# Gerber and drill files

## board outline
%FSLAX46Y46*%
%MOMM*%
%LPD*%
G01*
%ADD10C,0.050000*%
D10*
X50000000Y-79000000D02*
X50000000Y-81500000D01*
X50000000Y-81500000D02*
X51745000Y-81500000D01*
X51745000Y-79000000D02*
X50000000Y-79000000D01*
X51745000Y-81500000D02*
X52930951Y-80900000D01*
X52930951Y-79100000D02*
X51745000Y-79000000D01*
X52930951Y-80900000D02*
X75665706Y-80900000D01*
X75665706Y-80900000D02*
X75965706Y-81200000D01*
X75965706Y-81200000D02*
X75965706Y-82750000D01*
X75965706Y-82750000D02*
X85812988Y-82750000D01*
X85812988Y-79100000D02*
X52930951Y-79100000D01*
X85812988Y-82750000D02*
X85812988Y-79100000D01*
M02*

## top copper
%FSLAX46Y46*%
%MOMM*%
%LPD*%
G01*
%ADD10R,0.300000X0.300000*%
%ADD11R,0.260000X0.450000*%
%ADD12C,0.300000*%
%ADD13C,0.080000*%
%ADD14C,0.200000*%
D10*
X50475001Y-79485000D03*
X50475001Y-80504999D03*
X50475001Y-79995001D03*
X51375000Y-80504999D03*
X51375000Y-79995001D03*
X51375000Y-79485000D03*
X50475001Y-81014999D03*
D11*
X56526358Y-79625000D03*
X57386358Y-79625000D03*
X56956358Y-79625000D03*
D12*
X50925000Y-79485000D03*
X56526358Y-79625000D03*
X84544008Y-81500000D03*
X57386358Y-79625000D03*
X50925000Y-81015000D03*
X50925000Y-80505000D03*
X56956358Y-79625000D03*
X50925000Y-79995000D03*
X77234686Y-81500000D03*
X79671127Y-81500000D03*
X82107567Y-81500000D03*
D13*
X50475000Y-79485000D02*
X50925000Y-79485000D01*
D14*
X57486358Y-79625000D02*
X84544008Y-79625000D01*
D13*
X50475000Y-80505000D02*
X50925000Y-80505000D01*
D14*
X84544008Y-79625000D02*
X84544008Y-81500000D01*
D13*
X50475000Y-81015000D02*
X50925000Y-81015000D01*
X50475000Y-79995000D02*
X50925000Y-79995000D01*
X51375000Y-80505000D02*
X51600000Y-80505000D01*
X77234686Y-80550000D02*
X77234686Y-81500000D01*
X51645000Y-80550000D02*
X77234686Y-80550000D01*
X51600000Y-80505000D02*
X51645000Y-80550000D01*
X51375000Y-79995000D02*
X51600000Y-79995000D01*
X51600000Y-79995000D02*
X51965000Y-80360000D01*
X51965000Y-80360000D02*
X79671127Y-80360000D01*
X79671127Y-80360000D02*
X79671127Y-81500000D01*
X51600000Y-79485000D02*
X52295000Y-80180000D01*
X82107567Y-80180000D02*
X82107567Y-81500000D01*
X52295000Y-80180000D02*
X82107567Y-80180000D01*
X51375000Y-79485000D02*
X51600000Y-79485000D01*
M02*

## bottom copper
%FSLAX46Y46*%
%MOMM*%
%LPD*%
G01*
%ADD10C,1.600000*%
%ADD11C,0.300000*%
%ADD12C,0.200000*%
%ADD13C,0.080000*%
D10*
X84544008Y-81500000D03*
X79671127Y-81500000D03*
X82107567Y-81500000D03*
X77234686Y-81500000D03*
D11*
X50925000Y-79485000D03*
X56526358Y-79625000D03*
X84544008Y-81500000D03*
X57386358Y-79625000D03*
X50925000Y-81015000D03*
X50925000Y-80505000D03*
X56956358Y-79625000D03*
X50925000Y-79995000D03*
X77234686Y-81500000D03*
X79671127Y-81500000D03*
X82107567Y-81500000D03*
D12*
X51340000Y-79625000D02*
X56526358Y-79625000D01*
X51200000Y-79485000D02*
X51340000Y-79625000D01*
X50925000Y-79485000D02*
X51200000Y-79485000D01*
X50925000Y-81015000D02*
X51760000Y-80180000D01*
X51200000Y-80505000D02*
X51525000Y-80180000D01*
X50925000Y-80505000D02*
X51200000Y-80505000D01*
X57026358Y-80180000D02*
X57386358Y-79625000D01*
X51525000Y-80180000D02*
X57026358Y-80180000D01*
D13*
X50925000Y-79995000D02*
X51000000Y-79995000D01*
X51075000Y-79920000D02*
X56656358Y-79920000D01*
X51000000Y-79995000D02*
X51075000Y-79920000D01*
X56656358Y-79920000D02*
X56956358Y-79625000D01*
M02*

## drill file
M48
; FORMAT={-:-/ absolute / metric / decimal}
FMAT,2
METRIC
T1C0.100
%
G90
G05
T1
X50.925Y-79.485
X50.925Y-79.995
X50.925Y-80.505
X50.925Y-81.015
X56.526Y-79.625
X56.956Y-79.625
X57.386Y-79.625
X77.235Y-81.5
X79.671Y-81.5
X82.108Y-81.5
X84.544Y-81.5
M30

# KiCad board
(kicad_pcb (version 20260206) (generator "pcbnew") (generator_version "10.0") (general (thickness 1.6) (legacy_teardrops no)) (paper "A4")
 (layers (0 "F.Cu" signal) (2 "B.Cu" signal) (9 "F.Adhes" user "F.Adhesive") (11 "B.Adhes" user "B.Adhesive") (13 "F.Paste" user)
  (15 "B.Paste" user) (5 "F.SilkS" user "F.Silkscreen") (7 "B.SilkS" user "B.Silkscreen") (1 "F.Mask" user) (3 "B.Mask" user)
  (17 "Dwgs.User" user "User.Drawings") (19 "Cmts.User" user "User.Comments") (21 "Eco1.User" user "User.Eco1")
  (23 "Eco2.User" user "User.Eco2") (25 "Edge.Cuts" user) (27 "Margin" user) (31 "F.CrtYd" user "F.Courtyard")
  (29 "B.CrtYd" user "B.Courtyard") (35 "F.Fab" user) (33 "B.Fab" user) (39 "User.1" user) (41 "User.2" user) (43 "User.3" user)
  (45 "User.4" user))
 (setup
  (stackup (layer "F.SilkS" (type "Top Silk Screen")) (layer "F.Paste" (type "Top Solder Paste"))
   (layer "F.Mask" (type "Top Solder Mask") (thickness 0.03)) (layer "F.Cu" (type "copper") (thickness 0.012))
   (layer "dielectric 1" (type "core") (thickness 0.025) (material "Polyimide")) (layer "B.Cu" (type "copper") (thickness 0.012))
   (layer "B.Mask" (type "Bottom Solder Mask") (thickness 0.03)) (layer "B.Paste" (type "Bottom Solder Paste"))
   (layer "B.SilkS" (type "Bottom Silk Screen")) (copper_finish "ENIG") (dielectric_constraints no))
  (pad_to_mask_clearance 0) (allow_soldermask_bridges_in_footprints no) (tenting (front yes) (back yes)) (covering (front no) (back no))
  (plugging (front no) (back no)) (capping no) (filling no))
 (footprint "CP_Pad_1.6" (layer "F.Cu") (at 84.544008 81.5)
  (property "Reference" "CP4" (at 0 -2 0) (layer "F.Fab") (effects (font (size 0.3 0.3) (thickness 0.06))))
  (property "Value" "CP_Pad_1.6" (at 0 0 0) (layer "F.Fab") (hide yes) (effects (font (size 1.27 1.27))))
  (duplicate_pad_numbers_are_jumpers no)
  (pad "1" smd circle (at 0 0) (size 1.6 1.6) (layers "B.Cu" "B.Mask") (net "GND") (solder_mask_margin 0.1)))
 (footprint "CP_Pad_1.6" (layer "F.Cu") (at 77.234686 81.5)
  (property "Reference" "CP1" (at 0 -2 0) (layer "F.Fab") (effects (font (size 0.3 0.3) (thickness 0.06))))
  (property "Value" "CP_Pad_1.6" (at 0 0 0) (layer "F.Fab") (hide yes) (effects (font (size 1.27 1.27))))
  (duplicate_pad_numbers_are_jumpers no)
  (pad "1" smd circle (at 0 0) (size 1.6 1.6) (layers "B.Cu" "B.Mask") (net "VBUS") (solder_mask_margin 0.1)))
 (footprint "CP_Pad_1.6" (layer "F.Cu") (at 82.107567 81.5)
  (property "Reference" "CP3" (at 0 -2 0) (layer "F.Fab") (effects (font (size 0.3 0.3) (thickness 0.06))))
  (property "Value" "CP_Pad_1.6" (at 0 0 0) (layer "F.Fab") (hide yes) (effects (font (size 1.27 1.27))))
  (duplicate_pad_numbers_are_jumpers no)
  (pad "1" smd circle (at 0 0) (size 1.6 1.6) (layers "B.Cu" "B.Mask") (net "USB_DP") (solder_mask_margin 0.1)))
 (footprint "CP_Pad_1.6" (layer "F.Cu") (at 79.671127 81.5)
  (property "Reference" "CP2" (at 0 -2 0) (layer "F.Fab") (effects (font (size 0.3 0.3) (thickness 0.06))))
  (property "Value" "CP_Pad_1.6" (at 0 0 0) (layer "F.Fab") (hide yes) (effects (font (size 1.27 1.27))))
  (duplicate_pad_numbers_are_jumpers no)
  (pad "1" smd circle (at 0 0) (size 1.6 1.6) (layers "B.Cu" "B.Mask") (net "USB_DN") (solder_mask_margin 0.1)))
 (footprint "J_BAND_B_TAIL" (layer "F.Cu") (at 50.9 80.25)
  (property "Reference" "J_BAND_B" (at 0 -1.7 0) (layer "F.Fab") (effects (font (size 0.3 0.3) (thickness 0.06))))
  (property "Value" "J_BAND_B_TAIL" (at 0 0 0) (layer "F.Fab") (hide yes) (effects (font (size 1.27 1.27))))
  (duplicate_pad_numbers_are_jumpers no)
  (pad "1" smd rect (at -0.424999 -0.765) (size 0.3 0.3) (layers "F.Cu" "F.Mask") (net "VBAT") (solder_mask_margin 0.05)
   (thermal_bridge_angle 45))
  (pad "2" smd rect (at -0.424999 0.254999) (size 0.3 0.3) (layers "F.Cu" "F.Mask") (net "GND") (solder_mask_margin 0.05)
   (thermal_bridge_angle 45))
  (pad "3" smd rect (at -0.424999 -0.254999) (size 0.3 0.3) (layers "F.Cu" "F.Mask") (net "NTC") (solder_mask_margin 0.05)
   (thermal_bridge_angle 45))
  (pad "4" smd rect (at 0.475 0.254999) (size 0.3 0.3) (layers "F.Cu" "F.Mask") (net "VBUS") (solder_mask_margin 0.05)
   (thermal_bridge_angle 45))
  (pad "5" smd rect (at 0.475 -0.254999) (size 0.3 0.3) (layers "F.Cu" "F.Mask") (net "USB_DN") (solder_mask_margin 0.05)
   (thermal_bridge_angle 45))
  (pad "6" smd rect (at 0.475 -0.765) (size 0.3 0.3) (layers "F.Cu" "F.Mask") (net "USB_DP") (solder_mask_margin 0.05)
   (thermal_bridge_angle 45))
  (pad "7" smd rect (at -0.424999 0.764999) (size 0.3 0.3) (layers "F.Cu" "F.Mask") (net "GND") (solder_mask_margin 0.05)
   (thermal_bridge_angle 45)))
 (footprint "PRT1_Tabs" (layer "F.Cu") (at 56.956358 79.625)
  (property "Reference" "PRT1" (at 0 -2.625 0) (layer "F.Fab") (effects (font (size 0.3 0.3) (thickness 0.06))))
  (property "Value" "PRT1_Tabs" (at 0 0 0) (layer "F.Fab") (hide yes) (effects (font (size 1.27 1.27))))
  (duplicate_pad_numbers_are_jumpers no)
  (pad "1" smd rect (at -0.43 0) (size 0.26 0.45) (layers "F.Cu" "F.Mask") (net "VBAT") (solder_mask_margin 0.05) (thermal_bridge_angle 45))
  (pad "2" smd rect (at 0.43 0) (size 0.26 0.45) (layers "F.Cu" "F.Mask") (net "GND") (solder_mask_margin 0.05) (thermal_bridge_angle 45))
  (pad "3" smd rect (at 0 0) (size 0.26 0.45) (layers "F.Cu" "F.Mask") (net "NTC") (solder_mask_margin 0.05) (thermal_bridge_angle 45)))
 (gr_line (start 50 79) (end 50 81.5) (stroke (width 0.05) (type default)) (layer "Edge.Cuts"))
 (gr_line (start 50 81.5) (end 51.745 81.5) (stroke (width 0.05) (type default)) (layer "Edge.Cuts"))
 (gr_line (start 51.745 79) (end 50 79) (stroke (width 0.05) (type default)) (layer "Edge.Cuts"))
 (gr_line (start 51.745 81.5) (end 52.930951 80.9) (stroke (width 0.05) (type default)) (layer "Edge.Cuts"))
 (gr_line (start 52.930951 79.1) (end 51.745 79) (stroke (width 0.05) (type default)) (layer "Edge.Cuts"))
 (gr_line (start 52.930951 80.9) (end 75.665706 80.9) (stroke (width 0.05) (type default)) (layer "Edge.Cuts"))
 (gr_line (start 75.665706 80.9) (end 75.965706 81.2) (stroke (width 0.05) (type default)) (layer "Edge.Cuts"))
 (gr_line (start 75.965706 81.2) (end 75.965706 82.75) (stroke (width 0.05) (type default)) (layer "Edge.Cuts"))
 (gr_line (start 75.965706 82.75) (end 85.812988 82.75) (stroke (width 0.05) (type default)) (layer "Edge.Cuts"))
 (gr_line (start 85.812988 79.1) (end 52.930951 79.1) (stroke (width 0.05) (type default)) (layer "Edge.Cuts"))
 (gr_line (start 85.812988 82.75) (end 85.812988 79.1) (stroke (width 0.05) (type default)) (layer "Edge.Cuts"))
 (segment (start 50.475 79.485) (end 50.925 79.485) (width 0.08) (layer "F.Cu") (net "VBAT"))
 (via (at 56.526358 79.625) (size 0.3) (drill 0.1) (layers "F.Cu" "B.Cu") (tenting (front yes) (back yes)) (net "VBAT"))
 (via (at 50.925 79.485) (size 0.3) (drill 0.1) (layers "F.Cu" "B.Cu") (tenting (front yes) (back yes)) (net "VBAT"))
 (segment (start 50.925 79.485) (end 51.2 79.485) (width 0.2) (layer "B.Cu") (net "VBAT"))
 (segment (start 51.34 79.625) (end 56.526358 79.625) (width 0.2) (layer "B.Cu") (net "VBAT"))
 (segment (start 51.2 79.485) (end 51.34 79.625) (width 0.2) (layer "B.Cu") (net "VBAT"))
 (segment (start 50.475 81.015) (end 50.925 81.015) (width 0.08) (layer "F.Cu") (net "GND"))
 (segment (start 84.544008 79.625) (end 84.544008 81.5) (width 0.2) (layer "F.Cu") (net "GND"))
 (segment (start 50.475 80.505) (end 50.925 80.505) (width 0.08) (layer "F.Cu") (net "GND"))
 (segment (start 57.486358 79.625) (end 84.544008 79.625) (width 0.2) (layer "F.Cu") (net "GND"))
 (via (at 50.925 81.015) (size 0.3) (drill 0.1) (layers "F.Cu" "B.Cu") (tenting (front yes) (back yes)) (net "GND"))
 (via (at 57.386358 79.625) (size 0.3) (drill 0.1) (layers "F.Cu" "B.Cu") (tenting (front yes) (back yes)) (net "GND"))
 (via (at 84.544008 81.5) (size 0.3) (drill 0.1) (layers "F.Cu" "B.Cu") (tenting (front yes) (back yes)) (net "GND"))
 (via (at 50.925 80.505) (size 0.3) (drill 0.1) (layers "F.Cu" "B.Cu") (tenting (front yes) (back yes)) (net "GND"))
 (segment (start 50.925 81.015) (end 51.76 80.18) (width 0.2) (layer "B.Cu") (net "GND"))
 (segment (start 50.925 80.505) (end 51.2 80.505) (width 0.2) (layer "B.Cu") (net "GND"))
 (segment (start 51.525 80.18) (end 57.026358 80.18) (width 0.2) (layer "B.Cu") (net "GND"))
 (segment (start 57.026358 80.18) (end 57.386358 79.625) (width 0.2) (layer "B.Cu") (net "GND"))
 (segment (start 51.2 80.505) (end 51.525 80.18) (width 0.2) (layer "B.Cu") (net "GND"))
 (segment (start 50.475 79.995) (end 50.925 79.995) (width 0.08) (layer "F.Cu") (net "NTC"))
 (via (at 50.925 79.995) (size 0.3) (drill 0.1) (layers "F.Cu" "B.Cu") (tenting (front yes) (back yes)) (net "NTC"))
 (via (at 56.956358 79.625) (size 0.3) (drill 0.1) (layers "F.Cu" "B.Cu") (tenting (front yes) (back yes)) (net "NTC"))
 (segment (start 50.925 79.995) (end 51 79.995) (width 0.08) (layer "B.Cu") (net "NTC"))
 (segment (start 56.656358 79.92) (end 56.956358 79.625) (width 0.08) (layer "B.Cu") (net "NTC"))
 (segment (start 51 79.995) (end 51.075 79.92) (width 0.08) (layer "B.Cu") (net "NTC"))
 (segment (start 51.075 79.92) (end 56.656358 79.92) (width 0.08) (layer "B.Cu") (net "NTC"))
 (segment (start 77.234686 80.55) (end 77.234686 81.5) (width 0.08) (layer "F.Cu") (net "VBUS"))
 (segment (start 51.645 80.55) (end 77.234686 80.55) (width 0.08) (layer "F.Cu") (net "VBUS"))
 (segment (start 51.375 80.505) (end 51.6 80.505) (width 0.08) (layer "F.Cu") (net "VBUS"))
 (segment (start 51.6 80.505) (end 51.645 80.55) (width 0.08) (layer "F.Cu") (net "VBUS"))
 (via (at 77.234686 81.5) (size 0.3) (drill 0.1) (layers "F.Cu" "B.Cu") (tenting (front yes) (back yes)) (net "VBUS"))
 (segment (start 51.6 79.995) (end 51.965 80.36) (width 0.08) (layer "F.Cu") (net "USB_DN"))
 (segment (start 51.965 80.36) (end 79.671127 80.36) (width 0.08) (layer "F.Cu") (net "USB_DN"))
 (segment (start 51.375 79.995) (end 51.6 79.995) (width 0.08) (layer "F.Cu") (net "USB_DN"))
 (segment (start 79.671127 80.36) (end 79.671127 81.5) (width 0.08) (layer "F.Cu") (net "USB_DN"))
 (via (at 79.671127 81.5) (size 0.3) (drill 0.1) (layers "F.Cu" "B.Cu") (tenting (front yes) (back yes)) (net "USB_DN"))
 (segment (start 82.107567 80.18) (end 82.107567 81.5) (width 0.08) (layer "F.Cu") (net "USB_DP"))
 (segment (start 52.295 80.18) (end 82.107567 80.18) (width 0.08) (layer "F.Cu") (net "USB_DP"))
 (segment (start 51.375 79.485) (end 51.6 79.485) (width 0.08) (layer "F.Cu") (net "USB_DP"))
 (segment (start 51.6 79.485) (end 52.295 80.18) (width 0.08) (layer "F.Cu") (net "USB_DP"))
 (via (at 82.107567 81.5) (size 0.3) (drill 0.1) (layers "F.Cu" "B.Cu") (tenting (front yes) (back yes)) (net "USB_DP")))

